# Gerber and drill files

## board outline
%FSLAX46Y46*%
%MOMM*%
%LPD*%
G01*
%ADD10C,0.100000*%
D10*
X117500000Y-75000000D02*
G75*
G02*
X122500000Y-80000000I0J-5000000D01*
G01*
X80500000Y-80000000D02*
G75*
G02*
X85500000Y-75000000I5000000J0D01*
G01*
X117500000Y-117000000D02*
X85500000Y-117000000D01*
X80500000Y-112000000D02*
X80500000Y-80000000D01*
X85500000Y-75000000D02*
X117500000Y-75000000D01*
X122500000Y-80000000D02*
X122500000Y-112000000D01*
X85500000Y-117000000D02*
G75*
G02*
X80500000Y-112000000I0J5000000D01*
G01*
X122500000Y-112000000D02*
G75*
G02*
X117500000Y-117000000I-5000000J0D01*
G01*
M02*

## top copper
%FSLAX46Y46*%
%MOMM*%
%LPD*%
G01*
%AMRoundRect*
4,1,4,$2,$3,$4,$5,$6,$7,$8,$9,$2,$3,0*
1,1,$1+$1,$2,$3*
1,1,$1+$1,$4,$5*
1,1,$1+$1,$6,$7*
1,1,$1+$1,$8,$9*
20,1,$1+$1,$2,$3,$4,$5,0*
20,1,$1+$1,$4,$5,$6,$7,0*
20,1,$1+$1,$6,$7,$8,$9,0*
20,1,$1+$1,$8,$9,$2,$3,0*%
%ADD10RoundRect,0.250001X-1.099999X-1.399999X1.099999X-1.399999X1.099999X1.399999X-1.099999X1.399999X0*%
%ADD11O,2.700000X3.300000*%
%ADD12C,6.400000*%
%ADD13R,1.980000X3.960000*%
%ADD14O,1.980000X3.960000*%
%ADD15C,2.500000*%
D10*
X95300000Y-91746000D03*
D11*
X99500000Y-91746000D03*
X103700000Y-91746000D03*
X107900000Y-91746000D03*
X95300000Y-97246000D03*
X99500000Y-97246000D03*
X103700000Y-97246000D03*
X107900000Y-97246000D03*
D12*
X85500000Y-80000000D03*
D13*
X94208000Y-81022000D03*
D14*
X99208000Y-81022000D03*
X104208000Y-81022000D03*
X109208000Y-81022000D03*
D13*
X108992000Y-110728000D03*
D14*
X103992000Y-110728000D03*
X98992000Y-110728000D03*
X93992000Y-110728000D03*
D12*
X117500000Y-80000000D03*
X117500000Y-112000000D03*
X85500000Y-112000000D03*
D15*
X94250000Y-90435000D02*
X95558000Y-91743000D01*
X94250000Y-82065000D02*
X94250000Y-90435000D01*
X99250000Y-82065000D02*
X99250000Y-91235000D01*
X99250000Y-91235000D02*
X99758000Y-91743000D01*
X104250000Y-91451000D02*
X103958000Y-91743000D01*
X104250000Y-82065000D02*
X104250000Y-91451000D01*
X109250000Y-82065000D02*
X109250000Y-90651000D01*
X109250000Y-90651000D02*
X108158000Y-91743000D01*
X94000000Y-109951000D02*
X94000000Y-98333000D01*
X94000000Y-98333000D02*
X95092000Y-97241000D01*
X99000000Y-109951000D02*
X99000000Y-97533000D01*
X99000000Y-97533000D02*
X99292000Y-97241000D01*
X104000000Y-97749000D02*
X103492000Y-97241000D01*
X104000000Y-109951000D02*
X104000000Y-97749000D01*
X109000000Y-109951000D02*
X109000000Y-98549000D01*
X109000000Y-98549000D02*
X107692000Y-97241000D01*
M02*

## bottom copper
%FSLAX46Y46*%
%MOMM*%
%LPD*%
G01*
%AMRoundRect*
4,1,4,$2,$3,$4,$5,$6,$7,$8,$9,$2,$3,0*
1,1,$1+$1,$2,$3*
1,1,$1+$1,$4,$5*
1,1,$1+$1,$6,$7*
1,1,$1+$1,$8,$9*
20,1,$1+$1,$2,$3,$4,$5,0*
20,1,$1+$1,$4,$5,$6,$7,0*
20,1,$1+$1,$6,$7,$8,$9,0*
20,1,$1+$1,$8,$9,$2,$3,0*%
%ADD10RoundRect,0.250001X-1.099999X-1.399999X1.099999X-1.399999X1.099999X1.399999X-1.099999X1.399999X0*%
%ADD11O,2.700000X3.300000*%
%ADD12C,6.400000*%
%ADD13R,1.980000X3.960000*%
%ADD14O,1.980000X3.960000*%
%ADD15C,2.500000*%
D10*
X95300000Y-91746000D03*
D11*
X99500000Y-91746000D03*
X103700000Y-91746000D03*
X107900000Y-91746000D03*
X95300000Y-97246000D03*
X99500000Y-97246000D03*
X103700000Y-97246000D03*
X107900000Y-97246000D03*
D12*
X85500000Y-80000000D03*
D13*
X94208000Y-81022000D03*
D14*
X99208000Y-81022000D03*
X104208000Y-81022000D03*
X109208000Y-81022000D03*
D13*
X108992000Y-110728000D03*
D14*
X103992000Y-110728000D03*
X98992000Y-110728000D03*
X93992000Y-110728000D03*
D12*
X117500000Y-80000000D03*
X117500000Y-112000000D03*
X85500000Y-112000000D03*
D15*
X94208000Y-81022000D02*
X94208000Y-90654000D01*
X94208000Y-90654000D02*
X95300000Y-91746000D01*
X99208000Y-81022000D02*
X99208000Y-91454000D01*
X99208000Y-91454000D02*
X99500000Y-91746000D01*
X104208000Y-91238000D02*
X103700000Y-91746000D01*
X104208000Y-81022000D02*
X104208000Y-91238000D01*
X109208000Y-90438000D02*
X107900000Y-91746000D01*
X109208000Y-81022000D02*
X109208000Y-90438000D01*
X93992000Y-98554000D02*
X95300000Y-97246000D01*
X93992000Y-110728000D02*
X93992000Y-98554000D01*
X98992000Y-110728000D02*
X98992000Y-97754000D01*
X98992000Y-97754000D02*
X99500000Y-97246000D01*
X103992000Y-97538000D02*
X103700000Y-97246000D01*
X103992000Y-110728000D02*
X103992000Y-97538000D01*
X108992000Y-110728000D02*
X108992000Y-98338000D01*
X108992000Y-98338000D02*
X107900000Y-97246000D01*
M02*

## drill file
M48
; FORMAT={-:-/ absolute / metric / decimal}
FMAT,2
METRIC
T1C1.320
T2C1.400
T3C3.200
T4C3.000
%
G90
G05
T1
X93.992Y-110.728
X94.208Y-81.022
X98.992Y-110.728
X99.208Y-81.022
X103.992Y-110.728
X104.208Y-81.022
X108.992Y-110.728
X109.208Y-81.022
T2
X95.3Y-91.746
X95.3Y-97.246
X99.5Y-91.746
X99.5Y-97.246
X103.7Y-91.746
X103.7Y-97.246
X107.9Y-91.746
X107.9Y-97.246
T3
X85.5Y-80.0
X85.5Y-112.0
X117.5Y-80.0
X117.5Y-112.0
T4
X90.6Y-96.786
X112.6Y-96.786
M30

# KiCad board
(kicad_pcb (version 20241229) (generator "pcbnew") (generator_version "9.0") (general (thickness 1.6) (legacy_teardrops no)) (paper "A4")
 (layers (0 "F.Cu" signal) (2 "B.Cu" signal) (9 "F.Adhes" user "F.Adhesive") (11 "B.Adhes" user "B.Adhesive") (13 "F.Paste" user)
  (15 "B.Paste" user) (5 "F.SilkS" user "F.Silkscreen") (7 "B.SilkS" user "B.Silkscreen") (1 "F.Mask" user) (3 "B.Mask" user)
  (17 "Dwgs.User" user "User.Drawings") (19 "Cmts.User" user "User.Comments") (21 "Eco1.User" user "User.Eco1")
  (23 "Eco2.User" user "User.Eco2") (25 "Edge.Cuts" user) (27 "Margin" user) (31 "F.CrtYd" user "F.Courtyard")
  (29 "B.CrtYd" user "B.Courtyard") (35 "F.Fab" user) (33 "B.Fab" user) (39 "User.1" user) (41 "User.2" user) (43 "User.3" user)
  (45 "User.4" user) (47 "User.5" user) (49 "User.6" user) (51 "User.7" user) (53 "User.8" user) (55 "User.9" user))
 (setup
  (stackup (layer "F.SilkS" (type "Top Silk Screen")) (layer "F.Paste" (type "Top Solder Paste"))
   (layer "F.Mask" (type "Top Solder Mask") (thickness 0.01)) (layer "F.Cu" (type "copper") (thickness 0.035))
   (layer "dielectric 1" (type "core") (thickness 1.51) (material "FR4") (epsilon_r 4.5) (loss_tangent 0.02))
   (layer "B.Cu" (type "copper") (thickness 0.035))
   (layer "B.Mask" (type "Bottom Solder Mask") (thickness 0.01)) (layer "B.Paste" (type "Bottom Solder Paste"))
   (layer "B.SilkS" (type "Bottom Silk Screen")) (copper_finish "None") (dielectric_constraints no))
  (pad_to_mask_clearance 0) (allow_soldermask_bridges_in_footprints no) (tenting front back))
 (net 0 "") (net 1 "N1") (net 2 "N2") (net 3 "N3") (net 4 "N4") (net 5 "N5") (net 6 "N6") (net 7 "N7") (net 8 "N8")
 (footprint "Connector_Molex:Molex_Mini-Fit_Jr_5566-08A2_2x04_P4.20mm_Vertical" (layer "F.Cu") (at 95.3 91.746)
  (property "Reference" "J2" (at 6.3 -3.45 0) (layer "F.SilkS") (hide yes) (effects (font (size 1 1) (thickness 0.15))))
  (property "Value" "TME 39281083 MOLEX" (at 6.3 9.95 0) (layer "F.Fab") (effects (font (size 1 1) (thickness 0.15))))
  (pad "" np_thru_hole circle (at -4.7 5.04) (size 3 3) (drill 3) (layers "*.Cu" "*.Mask"))
  (pad "" np_thru_hole circle (at 17.3 5.04) (size 3 3) (drill 3) (layers "*.Cu" "*.Mask"))
  (pad "1" thru_hole roundrect (at 0 0) (size 2.7 3.3) (drill 1.4) (layers "*.Cu" "*.Mask") (remove_unused_layers no)
   (roundrect_rratio 0.092593) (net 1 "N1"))
  (pad "2" thru_hole oval (at 4.2 0) (size 2.7 3.3) (drill 1.4) (layers "*.Cu" "*.Mask") (remove_unused_layers no) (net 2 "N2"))
  (pad "3" thru_hole oval (at 8.4 0) (size 2.7 3.3) (drill 1.4) (layers "*.Cu" "*.Mask") (remove_unused_layers no) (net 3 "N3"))
  (pad "4" thru_hole oval (at 12.6 0) (size 2.7 3.3) (drill 1.4) (layers "*.Cu" "*.Mask") (remove_unused_layers no) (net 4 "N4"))
  (pad "5" thru_hole oval (at 0 5.5) (size 2.7 3.3) (drill 1.4) (layers "*.Cu" "*.Mask") (remove_unused_layers no) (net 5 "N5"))
  (pad "6" thru_hole oval (at 4.2 5.5) (size 2.7 3.3) (drill 1.4) (layers "*.Cu" "*.Mask") (remove_unused_layers no) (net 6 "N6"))
  (pad "7" thru_hole oval (at 8.4 5.5) (size 2.7 3.3) (drill 1.4) (layers "*.Cu" "*.Mask") (remove_unused_layers no) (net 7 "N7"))
  (pad "8" thru_hole oval (at 12.6 5.5) (size 2.7 3.3) (drill 1.4) (layers "*.Cu" "*.Mask") (remove_unused_layers no) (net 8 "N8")))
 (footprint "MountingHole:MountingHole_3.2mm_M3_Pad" (layer "F.Cu") (at 85.5 80)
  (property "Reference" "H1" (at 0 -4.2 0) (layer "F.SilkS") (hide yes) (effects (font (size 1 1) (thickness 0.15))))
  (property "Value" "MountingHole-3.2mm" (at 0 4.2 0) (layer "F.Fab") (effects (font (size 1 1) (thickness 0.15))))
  (pad "1" thru_hole circle (at 0 0) (size 6.4 6.4) (drill 3.2) (layers "*.Cu" "*.Mask") (remove_unused_layers no)))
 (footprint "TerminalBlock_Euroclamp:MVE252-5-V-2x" (layer "F.Cu") (at 101.6 81.25)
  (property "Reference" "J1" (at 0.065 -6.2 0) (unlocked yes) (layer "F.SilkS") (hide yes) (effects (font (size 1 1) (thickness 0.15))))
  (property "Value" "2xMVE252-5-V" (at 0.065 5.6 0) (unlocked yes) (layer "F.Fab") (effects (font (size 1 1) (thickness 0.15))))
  (pad "1" thru_hole rect (at -7.392 -0.228) (size 1.98 3.96) (drill 1.32) (layers "*.Cu" "*.Mask") (remove_unused_layers no) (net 1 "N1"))
  (pad "2" thru_hole oval (at -2.392 -0.228) (size 1.98 3.96) (drill 1.32) (layers "*.Cu" "*.Mask") (remove_unused_layers no) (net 2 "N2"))
  (pad "3" thru_hole oval (at 2.608 -0.228) (size 1.98 3.96) (drill 1.32) (layers "*.Cu" "*.Mask") (remove_unused_layers no) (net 3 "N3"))
  (pad "4" thru_hole oval (at 7.608 -0.228) (size 1.98 3.96) (drill 1.32) (layers "*.Cu" "*.Mask") (remove_unused_layers no) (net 4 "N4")))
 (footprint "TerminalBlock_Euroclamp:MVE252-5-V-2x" (layer "F.Cu") (at 101.6 110.5 180)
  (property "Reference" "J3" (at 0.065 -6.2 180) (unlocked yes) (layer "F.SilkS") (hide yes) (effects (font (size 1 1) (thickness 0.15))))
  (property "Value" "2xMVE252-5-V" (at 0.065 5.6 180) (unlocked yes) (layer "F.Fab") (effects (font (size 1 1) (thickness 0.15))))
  (pad "1" thru_hole rect (at -7.392 -0.228 180) (size 1.98 3.96) (drill 1.32) (layers "*.Cu" "*.Mask") (remove_unused_layers no)
   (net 8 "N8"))
  (pad "2" thru_hole oval (at -2.392 -0.228 180) (size 1.98 3.96) (drill 1.32) (layers "*.Cu" "*.Mask") (remove_unused_layers no)
   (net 7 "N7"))
  (pad "3" thru_hole oval (at 2.608 -0.228 180) (size 1.98 3.96) (drill 1.32) (layers "*.Cu" "*.Mask") (remove_unused_layers no)
   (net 6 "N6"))
  (pad "4" thru_hole oval (at 7.608 -0.228 180) (size 1.98 3.96) (drill 1.32) (layers "*.Cu" "*.Mask") (remove_unused_layers no)
   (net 5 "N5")))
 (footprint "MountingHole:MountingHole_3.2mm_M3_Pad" (layer "F.Cu") (at 117.5 80)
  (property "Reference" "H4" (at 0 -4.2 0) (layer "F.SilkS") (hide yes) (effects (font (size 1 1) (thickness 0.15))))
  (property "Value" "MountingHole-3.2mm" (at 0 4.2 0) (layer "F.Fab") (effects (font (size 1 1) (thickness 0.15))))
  (pad "1" thru_hole circle (at 0 0) (size 6.4 6.4) (drill 3.2) (layers "*.Cu" "*.Mask") (remove_unused_layers no)))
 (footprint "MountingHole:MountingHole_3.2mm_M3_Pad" (layer "F.Cu") (at 117.5 112)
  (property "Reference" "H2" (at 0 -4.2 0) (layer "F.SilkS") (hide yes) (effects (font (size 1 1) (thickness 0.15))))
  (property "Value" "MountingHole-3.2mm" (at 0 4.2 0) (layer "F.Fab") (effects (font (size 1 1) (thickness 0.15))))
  (pad "1" thru_hole circle (at 0 0) (size 6.4 6.4) (drill 3.2) (layers "*.Cu" "*.Mask") (remove_unused_layers no)))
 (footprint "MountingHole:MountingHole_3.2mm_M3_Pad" (layer "F.Cu") (at 85.5 112)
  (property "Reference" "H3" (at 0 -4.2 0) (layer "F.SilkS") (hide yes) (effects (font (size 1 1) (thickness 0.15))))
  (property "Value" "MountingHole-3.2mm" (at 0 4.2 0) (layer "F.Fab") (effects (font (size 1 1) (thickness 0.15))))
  (pad "1" thru_hole circle (at 0 0) (size 6.4 6.4) (drill 3.2) (layers "*.Cu" "*.Mask") (remove_unused_layers no)))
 (gr_arc (start 117.5 75) (mid 121.035534 76.464466) (end 122.5 80) (stroke (width 0.1) (type solid)) (layer "Edge.Cuts"))
 (gr_arc (start 80.5 80) (mid 81.964466 76.464466) (end 85.5 75) (stroke (width 0.1) (type solid)) (layer "Edge.Cuts"))
 (gr_line (start 117.5 117) (end 85.5 117) (stroke (width 0.1) (type solid)) (layer "Edge.Cuts"))
 (gr_line (start 80.5 112) (end 80.5 80) (stroke (width 0.1) (type solid)) (layer "Edge.Cuts"))
 (gr_line (start 85.5 75) (end 117.5 75) (stroke (width 0.1) (type solid)) (layer "Edge.Cuts"))
 (gr_line (start 122.5 80) (end 122.5 112) (stroke (width 0.1) (type solid)) (layer "Edge.Cuts"))
 (gr_arc (start 85.5 117) (mid 81.964466 115.535534) (end 80.5 112) (stroke (width 0.1) (type solid)) (layer "Edge.Cuts"))
 (gr_arc (start 122.5 112) (mid 121.035534 115.535534) (end 117.5 117) (stroke (width 0.1) (type solid)) (layer "Edge.Cuts"))
 (segment (start 94.25 90.435) (end 95.558 91.743) (width 2.5) (layer "F.Cu") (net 1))
 (segment (start 94.25 82.065) (end 94.25 90.435) (width 2.5) (layer "F.Cu") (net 1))
 (segment (start 94.208 81.022) (end 94.208 90.654) (width 2.5) (layer "B.Cu") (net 1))
 (segment (start 94.208 90.654) (end 95.3 91.746) (width 2.5) (layer "B.Cu") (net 1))
 (segment (start 99.25 82.065) (end 99.25 91.235) (width 2.5) (layer "F.Cu") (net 2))
 (segment (start 99.25 91.235) (end 99.758 91.743) (width 2.5) (layer "F.Cu") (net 2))
 (segment (start 99.208 81.022) (end 99.208 91.454) (width 2.5) (layer "B.Cu") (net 2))
 (segment (start 99.208 91.454) (end 99.5 91.746) (width 2.5) (layer "B.Cu") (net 2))
 (segment (start 104.25 91.451) (end 103.958 91.743) (width 2.5) (layer "F.Cu") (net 3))
 (segment (start 104.25 82.065) (end 104.25 91.451) (width 2.5) (layer "F.Cu") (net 3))
 (segment (start 104.208 91.238) (end 103.7 91.746) (width 2.5) (layer "B.Cu") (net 3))
 (segment (start 104.208 81.022) (end 104.208 91.238) (width 2.5) (layer "B.Cu") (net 3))
 (segment (start 109.25 82.065) (end 109.25 90.651) (width 2.5) (layer "F.Cu") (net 4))
 (segment (start 109.25 90.651) (end 108.158 91.743) (width 2.5) (layer "F.Cu") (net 4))
 (segment (start 109.208 90.438) (end 107.9 91.746) (width 2.5) (layer "B.Cu") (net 4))
 (segment (start 109.208 81.022) (end 109.208 90.438) (width 2.5) (layer "B.Cu") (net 4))
 (segment (start 94 109.951) (end 94 98.333) (width 2.5) (layer "F.Cu") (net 5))
 (segment (start 94 98.333) (end 95.092 97.241) (width 2.5) (layer "F.Cu") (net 5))
 (segment (start 93.992 98.554) (end 95.3 97.246) (width 2.5) (layer "B.Cu") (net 5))
 (segment (start 93.992 110.728) (end 93.992 98.554) (width 2.5) (layer "B.Cu") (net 5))
 (segment (start 99 109.951) (end 99 97.533) (width 2.5) (layer "F.Cu") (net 6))
 (segment (start 99 97.533) (end 99.292 97.241) (width 2.5) (layer "F.Cu") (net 6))
 (segment (start 98.992 110.728) (end 98.992 97.754) (width 2.5) (layer "B.Cu") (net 6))
 (segment (start 98.992 97.754) (end 99.5 97.246) (width 2.5) (layer "B.Cu") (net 6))
 (segment (start 104 97.749) (end 103.492 97.241) (width 2.5) (layer "F.Cu") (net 7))
 (segment (start 104 109.951) (end 104 97.749) (width 2.5) (layer "F.Cu") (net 7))
 (segment (start 103.992 97.538) (end 103.7 97.246) (width 2.5) (layer "B.Cu") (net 7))
 (segment (start 103.992 110.728) (end 103.992 97.538) (width 2.5) (layer "B.Cu") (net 7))
 (segment (start 109 109.951) (end 109 98.549) (width 2.5) (layer "F.Cu") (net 8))
 (segment (start 109 98.549) (end 107.692 97.241) (width 2.5) (layer "F.Cu") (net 8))
 (segment (start 108.992 110.728) (end 108.992 98.338) (width 2.5) (layer "B.Cu") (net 8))
 (segment (start 108.992 98.338) (end 107.9 97.246) (width 2.5) (layer "B.Cu") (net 8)))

